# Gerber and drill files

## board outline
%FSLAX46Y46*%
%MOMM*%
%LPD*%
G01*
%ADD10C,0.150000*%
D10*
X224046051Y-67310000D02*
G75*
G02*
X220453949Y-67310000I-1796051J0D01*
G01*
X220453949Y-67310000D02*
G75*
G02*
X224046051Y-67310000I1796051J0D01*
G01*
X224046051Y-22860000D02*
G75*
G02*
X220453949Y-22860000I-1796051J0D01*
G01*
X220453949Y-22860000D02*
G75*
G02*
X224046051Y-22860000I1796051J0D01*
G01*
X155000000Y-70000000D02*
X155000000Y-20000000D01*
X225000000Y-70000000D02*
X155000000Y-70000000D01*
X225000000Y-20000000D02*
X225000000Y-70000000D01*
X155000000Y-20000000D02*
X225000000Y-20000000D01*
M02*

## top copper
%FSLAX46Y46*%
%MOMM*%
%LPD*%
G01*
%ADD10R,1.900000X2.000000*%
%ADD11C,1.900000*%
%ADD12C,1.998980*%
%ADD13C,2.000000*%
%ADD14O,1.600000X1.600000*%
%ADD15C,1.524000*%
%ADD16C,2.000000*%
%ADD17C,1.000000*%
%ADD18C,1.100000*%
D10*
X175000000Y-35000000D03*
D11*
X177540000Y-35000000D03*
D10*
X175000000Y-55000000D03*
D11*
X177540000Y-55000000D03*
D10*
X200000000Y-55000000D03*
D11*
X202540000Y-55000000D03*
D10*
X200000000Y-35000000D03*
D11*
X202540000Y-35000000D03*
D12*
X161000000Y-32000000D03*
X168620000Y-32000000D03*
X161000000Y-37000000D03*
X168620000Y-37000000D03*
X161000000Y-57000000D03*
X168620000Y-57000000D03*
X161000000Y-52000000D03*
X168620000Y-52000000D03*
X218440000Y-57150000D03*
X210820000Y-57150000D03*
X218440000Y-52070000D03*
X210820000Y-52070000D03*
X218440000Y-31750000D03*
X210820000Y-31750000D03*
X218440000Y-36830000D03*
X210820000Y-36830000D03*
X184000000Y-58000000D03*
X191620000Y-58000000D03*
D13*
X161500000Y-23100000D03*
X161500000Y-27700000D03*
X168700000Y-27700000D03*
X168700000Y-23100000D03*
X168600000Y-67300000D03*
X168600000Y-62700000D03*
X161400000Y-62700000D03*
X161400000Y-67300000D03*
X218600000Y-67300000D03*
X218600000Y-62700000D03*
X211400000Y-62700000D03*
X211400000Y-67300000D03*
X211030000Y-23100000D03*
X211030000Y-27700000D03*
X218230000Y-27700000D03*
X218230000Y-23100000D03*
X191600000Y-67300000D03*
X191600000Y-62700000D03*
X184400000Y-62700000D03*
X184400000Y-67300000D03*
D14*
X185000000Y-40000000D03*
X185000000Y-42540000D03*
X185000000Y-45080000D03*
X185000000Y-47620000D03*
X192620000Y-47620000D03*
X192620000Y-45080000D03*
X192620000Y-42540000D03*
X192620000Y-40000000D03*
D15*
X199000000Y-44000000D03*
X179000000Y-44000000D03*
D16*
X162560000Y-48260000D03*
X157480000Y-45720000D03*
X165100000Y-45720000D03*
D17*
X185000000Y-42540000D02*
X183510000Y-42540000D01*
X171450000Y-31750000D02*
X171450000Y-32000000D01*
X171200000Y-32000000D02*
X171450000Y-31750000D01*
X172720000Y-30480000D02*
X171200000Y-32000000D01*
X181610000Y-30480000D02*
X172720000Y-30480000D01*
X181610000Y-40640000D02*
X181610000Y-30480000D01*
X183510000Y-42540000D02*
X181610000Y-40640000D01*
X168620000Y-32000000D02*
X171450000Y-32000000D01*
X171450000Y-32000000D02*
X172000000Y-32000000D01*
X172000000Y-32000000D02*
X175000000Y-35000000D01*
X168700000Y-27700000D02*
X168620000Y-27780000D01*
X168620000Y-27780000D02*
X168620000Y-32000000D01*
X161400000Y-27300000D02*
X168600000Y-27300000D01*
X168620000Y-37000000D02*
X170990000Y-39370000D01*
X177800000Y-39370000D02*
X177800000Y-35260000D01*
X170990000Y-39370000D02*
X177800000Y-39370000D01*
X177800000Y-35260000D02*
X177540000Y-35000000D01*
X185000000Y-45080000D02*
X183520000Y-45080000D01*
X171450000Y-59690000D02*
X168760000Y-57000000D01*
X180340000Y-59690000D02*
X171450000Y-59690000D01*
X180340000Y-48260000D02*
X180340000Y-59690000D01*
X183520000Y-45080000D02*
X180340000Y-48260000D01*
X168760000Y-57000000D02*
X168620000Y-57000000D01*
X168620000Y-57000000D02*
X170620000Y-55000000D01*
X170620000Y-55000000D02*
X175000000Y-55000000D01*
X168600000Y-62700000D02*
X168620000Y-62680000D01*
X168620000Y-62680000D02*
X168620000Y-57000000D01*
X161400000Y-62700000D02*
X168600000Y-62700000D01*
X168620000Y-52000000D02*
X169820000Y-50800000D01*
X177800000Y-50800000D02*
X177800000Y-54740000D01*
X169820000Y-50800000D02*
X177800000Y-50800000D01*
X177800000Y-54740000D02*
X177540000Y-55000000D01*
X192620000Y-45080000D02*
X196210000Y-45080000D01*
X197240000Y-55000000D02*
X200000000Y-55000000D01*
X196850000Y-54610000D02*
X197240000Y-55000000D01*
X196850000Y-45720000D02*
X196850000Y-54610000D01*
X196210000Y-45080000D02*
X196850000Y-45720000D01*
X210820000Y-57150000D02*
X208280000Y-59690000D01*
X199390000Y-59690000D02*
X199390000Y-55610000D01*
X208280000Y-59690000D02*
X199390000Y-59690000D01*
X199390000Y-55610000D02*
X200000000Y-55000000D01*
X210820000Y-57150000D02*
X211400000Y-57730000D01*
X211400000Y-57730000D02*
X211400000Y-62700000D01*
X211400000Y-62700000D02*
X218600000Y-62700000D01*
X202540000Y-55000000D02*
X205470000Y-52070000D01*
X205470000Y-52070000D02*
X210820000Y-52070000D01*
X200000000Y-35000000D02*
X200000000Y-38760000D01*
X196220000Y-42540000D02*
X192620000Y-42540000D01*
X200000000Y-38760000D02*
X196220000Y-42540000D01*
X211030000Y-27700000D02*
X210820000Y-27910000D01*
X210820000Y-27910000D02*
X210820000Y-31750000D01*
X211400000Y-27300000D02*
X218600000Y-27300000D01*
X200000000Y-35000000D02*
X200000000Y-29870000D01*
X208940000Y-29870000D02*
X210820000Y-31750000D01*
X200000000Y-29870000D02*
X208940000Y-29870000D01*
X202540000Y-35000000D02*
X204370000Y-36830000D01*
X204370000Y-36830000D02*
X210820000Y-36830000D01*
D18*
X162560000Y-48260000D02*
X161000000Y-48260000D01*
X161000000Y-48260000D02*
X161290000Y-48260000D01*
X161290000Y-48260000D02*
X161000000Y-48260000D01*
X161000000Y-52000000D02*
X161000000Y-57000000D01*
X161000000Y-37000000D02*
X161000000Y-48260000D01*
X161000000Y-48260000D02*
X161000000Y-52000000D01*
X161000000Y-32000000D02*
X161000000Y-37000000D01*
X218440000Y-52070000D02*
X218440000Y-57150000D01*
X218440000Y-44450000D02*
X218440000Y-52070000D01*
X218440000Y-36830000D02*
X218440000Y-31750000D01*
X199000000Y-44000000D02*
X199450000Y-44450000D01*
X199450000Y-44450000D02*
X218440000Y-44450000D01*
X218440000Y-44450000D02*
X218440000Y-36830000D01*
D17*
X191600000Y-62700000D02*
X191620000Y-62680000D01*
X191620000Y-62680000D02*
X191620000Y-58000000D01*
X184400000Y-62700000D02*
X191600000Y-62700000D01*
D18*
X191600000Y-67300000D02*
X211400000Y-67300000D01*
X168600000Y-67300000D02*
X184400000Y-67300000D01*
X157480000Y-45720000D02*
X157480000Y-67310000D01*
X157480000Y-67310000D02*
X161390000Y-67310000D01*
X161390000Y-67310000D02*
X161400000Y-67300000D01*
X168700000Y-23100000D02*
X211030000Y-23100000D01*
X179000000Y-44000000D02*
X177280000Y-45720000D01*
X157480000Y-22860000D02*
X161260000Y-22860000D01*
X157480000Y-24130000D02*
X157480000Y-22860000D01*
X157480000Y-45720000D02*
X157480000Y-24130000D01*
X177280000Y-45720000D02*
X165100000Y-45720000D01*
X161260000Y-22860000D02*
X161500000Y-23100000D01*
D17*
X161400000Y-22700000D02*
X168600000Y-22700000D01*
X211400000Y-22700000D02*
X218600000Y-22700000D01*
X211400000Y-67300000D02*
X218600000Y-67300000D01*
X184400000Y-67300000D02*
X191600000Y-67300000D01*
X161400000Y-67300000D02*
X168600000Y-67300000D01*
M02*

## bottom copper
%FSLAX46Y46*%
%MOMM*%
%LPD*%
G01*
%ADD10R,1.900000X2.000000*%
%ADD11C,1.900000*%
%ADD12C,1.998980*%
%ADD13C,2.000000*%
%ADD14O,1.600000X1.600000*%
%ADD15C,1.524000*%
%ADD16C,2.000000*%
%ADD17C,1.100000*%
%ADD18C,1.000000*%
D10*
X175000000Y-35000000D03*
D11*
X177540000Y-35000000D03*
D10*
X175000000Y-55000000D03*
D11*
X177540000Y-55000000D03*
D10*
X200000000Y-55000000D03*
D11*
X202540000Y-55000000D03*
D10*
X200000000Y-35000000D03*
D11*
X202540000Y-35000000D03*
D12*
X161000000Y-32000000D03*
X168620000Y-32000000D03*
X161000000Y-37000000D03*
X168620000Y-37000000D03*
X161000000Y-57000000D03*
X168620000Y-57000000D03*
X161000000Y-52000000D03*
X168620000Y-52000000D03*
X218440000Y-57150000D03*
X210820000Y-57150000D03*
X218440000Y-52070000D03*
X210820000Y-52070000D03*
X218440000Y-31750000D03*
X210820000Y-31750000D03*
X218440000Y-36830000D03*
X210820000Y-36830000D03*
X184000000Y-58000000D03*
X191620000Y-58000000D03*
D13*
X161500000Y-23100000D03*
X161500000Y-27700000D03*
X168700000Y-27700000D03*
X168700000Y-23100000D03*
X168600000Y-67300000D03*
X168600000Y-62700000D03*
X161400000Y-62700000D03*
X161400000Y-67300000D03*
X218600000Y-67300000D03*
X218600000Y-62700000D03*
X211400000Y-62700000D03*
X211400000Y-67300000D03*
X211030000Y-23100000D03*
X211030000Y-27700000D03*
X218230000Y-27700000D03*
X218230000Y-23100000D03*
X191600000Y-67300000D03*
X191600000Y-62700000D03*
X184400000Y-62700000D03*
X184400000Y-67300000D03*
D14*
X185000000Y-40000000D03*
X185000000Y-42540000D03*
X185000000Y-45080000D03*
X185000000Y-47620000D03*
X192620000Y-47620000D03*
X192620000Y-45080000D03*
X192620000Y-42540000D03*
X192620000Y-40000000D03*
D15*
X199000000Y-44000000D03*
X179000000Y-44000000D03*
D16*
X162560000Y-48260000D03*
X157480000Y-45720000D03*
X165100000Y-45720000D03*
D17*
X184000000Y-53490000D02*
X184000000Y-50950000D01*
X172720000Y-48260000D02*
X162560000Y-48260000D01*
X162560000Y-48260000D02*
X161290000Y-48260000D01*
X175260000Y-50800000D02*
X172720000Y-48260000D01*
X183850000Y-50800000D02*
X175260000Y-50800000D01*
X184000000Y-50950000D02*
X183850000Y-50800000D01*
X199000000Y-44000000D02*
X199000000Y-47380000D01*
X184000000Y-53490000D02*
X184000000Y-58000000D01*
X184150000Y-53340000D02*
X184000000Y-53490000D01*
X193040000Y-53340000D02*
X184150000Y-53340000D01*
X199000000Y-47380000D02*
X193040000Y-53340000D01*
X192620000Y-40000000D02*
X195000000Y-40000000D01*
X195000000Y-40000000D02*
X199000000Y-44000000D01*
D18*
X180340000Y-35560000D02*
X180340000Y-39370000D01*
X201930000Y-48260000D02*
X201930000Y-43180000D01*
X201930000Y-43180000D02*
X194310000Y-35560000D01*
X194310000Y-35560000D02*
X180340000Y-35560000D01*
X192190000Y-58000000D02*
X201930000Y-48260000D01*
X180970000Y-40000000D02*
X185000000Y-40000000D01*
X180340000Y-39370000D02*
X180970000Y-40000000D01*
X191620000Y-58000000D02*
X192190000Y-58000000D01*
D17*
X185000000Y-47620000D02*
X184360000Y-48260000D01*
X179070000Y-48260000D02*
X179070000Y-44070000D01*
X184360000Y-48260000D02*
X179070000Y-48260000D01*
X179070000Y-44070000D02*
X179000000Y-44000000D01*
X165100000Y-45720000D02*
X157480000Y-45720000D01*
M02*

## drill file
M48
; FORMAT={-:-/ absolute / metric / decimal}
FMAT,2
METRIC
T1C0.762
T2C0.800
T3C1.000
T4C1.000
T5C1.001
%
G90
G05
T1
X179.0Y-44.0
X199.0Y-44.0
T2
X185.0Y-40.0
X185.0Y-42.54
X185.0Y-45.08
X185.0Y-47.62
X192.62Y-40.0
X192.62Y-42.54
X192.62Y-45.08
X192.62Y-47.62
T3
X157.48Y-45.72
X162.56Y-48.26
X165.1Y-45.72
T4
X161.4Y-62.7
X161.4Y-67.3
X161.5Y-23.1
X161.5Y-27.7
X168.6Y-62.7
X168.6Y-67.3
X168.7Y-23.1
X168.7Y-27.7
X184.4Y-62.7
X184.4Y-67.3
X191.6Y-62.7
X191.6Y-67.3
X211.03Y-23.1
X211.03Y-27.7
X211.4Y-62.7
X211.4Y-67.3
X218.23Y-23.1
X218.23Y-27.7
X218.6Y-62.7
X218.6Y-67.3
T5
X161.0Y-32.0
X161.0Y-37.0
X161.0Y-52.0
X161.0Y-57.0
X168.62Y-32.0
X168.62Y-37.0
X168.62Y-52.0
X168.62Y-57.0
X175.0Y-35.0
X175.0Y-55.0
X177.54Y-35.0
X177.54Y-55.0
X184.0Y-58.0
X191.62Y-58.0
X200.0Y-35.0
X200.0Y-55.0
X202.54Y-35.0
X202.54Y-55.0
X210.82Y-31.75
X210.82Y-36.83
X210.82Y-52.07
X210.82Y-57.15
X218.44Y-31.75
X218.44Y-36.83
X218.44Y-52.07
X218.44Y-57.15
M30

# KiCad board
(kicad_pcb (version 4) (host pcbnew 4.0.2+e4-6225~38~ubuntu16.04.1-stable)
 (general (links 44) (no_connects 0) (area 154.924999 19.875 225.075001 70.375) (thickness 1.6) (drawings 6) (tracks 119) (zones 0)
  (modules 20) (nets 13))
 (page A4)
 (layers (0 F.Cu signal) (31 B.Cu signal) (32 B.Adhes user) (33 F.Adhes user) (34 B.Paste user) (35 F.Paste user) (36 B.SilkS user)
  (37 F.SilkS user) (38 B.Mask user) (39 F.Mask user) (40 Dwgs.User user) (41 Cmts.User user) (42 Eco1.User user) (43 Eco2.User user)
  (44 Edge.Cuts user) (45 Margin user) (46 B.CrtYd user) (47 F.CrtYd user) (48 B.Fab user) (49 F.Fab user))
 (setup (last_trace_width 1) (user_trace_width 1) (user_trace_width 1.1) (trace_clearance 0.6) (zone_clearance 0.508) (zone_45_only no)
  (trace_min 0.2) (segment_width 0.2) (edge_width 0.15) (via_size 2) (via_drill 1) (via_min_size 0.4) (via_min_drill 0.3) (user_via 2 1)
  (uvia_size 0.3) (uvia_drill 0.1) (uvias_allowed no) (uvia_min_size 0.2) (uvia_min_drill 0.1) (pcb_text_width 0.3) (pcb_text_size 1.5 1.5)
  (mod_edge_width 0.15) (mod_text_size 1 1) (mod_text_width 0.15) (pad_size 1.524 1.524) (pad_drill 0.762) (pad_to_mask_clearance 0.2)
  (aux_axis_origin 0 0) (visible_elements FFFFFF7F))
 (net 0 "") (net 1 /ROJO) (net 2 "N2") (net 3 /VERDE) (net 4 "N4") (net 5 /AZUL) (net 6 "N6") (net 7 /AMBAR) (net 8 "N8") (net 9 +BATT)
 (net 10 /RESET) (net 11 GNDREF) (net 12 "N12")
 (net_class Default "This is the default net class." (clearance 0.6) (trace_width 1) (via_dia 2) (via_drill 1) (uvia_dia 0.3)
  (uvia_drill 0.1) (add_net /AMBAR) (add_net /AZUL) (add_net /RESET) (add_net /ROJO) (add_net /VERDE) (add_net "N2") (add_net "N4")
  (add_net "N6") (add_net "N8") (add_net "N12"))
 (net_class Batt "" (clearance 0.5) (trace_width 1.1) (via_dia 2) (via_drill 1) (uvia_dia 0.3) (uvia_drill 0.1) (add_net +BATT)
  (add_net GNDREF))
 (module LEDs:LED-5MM (layer F.Cu) (at 175 35)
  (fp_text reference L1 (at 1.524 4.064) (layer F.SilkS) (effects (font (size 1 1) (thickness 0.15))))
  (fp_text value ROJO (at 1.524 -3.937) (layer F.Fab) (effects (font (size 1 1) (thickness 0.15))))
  (pad 1 thru_hole rect (at 0 0 90) (size 2 1.9) (drill 1.00076) (layers *.Cu *.Mask F.SilkS) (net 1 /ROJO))
  (pad 2 thru_hole circle (at 2.54 0) (size 1.9 1.9) (drill 1.00076) (layers *.Cu *.Mask F.SilkS) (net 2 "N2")))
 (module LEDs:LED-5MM (layer F.Cu) (at 175 55)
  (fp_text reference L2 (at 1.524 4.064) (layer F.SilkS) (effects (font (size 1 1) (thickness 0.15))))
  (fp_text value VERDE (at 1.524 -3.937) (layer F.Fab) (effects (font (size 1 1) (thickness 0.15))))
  (pad 1 thru_hole rect (at 0 0 90) (size 2 1.9) (drill 1.00076) (layers *.Cu *.Mask F.SilkS) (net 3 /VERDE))
  (pad 2 thru_hole circle (at 2.54 0) (size 1.9 1.9) (drill 1.00076) (layers *.Cu *.Mask F.SilkS) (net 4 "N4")))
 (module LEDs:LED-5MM (layer F.Cu) (at 200 55)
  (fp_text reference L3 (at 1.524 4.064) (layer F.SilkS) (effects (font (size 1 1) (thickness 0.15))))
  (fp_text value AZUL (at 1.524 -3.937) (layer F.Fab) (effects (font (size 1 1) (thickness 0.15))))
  (pad 1 thru_hole rect (at 0 0 90) (size 2 1.9) (drill 1.00076) (layers *.Cu *.Mask F.SilkS) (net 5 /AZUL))
  (pad 2 thru_hole circle (at 2.54 0) (size 1.9 1.9) (drill 1.00076) (layers *.Cu *.Mask F.SilkS) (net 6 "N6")))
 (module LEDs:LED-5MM (layer F.Cu) (at 200 35)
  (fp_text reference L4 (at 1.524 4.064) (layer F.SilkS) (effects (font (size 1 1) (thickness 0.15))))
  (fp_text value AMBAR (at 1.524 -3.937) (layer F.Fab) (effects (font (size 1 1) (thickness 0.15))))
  (pad 1 thru_hole rect (at 0 0 90) (size 2 1.9) (drill 1.00076) (layers *.Cu *.Mask F.SilkS) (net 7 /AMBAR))
  (pad 2 thru_hole circle (at 2.54 0) (size 1.9 1.9) (drill 1.00076) (layers *.Cu *.Mask F.SilkS) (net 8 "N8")))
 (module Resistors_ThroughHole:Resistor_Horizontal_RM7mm (layer F.Cu) (at 161 32)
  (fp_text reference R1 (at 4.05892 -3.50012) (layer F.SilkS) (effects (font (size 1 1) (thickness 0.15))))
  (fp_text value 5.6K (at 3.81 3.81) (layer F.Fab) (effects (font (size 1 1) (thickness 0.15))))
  (pad 1 thru_hole circle (at 0 0) (size 1.99898 1.99898) (drill 1.00076) (layers *.Cu *.SilkS *.Mask) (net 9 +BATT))
  (pad 2 thru_hole circle (at 7.62 0) (size 1.99898 1.99898) (drill 1.00076) (layers *.Cu *.SilkS *.Mask) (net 1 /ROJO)))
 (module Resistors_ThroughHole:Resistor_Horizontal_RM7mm (layer F.Cu) (at 161 37)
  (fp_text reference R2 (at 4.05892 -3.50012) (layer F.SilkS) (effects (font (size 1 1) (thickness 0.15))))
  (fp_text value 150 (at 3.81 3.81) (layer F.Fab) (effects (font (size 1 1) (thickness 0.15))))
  (pad 1 thru_hole circle (at 0 0) (size 1.99898 1.99898) (drill 1.00076) (layers *.Cu *.SilkS *.Mask) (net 9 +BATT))
  (pad 2 thru_hole circle (at 7.62 0) (size 1.99898 1.99898) (drill 1.00076) (layers *.Cu *.SilkS *.Mask) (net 2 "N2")))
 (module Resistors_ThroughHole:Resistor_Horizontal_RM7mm (layer F.Cu) (at 161 57)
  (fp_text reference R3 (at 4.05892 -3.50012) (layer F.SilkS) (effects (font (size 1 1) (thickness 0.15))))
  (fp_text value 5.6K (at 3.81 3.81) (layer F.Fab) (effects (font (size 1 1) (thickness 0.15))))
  (pad 1 thru_hole circle (at 0 0) (size 1.99898 1.99898) (drill 1.00076) (layers *.Cu *.SilkS *.Mask) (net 9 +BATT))
  (pad 2 thru_hole circle (at 7.62 0) (size 1.99898 1.99898) (drill 1.00076) (layers *.Cu *.SilkS *.Mask) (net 3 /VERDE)))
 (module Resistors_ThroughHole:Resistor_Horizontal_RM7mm (layer F.Cu) (at 161 52)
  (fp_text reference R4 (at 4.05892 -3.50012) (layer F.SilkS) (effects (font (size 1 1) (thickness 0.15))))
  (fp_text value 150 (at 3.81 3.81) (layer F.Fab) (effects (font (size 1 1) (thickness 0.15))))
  (pad 1 thru_hole circle (at 0 0) (size 1.99898 1.99898) (drill 1.00076) (layers *.Cu *.SilkS *.Mask) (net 9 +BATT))
  (pad 2 thru_hole circle (at 7.62 0) (size 1.99898 1.99898) (drill 1.00076) (layers *.Cu *.SilkS *.Mask) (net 4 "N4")))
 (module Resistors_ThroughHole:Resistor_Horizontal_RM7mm (layer F.Cu) (at 218.44 57.15 180)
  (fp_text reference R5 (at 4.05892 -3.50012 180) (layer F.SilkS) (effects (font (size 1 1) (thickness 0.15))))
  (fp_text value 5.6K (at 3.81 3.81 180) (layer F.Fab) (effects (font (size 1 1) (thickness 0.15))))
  (pad 1 thru_hole circle (at 0 0 180) (size 1.99898 1.99898) (drill 1.00076) (layers *.Cu *.SilkS *.Mask) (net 9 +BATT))
  (pad 2 thru_hole circle (at 7.62 0 180) (size 1.99898 1.99898) (drill 1.00076) (layers *.Cu *.SilkS *.Mask) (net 5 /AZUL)))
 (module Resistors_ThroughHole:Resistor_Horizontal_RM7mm (layer F.Cu) (at 218.44 52.07 180)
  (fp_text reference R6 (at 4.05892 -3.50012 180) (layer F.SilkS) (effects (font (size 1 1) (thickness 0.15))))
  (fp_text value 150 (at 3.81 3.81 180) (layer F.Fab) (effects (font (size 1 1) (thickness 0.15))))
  (pad 1 thru_hole circle (at 0 0 180) (size 1.99898 1.99898) (drill 1.00076) (layers *.Cu *.SilkS *.Mask) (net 9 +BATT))
  (pad 2 thru_hole circle (at 7.62 0 180) (size 1.99898 1.99898) (drill 1.00076) (layers *.Cu *.SilkS *.Mask) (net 6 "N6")))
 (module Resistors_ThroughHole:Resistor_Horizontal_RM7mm (layer F.Cu) (at 218.44 31.75 180)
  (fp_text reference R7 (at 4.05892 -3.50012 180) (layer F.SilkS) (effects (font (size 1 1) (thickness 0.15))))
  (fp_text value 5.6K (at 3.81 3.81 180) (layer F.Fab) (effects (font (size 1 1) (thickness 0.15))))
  (pad 1 thru_hole circle (at 0 0 180) (size 1.99898 1.99898) (drill 1.00076) (layers *.Cu *.SilkS *.Mask) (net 9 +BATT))
  (pad 2 thru_hole circle (at 7.62 0 180) (size 1.99898 1.99898) (drill 1.00076) (layers *.Cu *.SilkS *.Mask) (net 7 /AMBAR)))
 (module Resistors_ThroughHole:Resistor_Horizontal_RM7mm (layer F.Cu) (at 218.44 36.83 180)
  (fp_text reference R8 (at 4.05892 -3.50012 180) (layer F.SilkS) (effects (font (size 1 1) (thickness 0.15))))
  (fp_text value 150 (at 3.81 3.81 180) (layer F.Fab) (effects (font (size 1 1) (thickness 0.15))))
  (pad 1 thru_hole circle (at 0 0 180) (size 1.99898 1.99898) (drill 1.00076) (layers *.Cu *.SilkS *.Mask) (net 9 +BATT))
  (pad 2 thru_hole circle (at 7.62 0 180) (size 1.99898 1.99898) (drill 1.00076) (layers *.Cu *.SilkS *.Mask) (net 8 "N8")))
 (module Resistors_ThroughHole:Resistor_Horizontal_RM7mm (layer F.Cu) (at 184 58)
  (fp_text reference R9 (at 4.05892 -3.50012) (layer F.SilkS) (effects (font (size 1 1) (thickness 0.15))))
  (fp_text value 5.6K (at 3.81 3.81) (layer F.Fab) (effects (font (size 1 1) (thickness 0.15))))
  (pad 1 thru_hole circle (at 0 0) (size 1.99898 1.99898) (drill 1.00076) (layers *.Cu *.SilkS *.Mask) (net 9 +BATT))
  (pad 2 thru_hole circle (at 7.62 0) (size 1.99898 1.99898) (drill 1.00076) (layers *.Cu *.SilkS *.Mask) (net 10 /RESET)))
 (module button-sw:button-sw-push (layer F.Cu) (at 165.1 25.4 180)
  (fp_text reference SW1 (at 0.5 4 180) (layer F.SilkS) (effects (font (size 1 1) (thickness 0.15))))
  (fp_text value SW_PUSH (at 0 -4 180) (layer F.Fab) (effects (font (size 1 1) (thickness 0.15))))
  (pad 1 thru_hole circle (at 3.6 2.3 180) (size 2 2) (drill 1) (layers *.Cu *.Mask F.SilkS) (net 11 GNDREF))
  (pad 2 thru_hole circle (at 3.6 -2.3 180) (size 2 2) (drill 1) (layers *.Cu *.Mask F.SilkS) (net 1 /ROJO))
  (pad 2 thru_hole circle (at -3.6 -2.3 180) (size 2 2) (drill 1) (layers *.Cu *.Mask F.SilkS) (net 1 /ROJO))
  (pad 1 thru_hole circle (at -3.6 2.3 180) (size 2 2) (drill 1) (layers *.Cu *.Mask F.SilkS) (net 11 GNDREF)))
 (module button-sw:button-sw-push (layer F.Cu) (at 165 65)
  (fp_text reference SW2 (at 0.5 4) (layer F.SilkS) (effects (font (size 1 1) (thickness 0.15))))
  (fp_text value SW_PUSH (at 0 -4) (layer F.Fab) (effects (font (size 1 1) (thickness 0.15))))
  (pad 1 thru_hole circle (at 3.6 2.3) (size 2 2) (drill 1) (layers *.Cu *.Mask F.SilkS) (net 11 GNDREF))
  (pad 2 thru_hole circle (at 3.6 -2.3) (size 2 2) (drill 1) (layers *.Cu *.Mask F.SilkS) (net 3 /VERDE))
  (pad 2 thru_hole circle (at -3.6 -2.3) (size 2 2) (drill 1) (layers *.Cu *.Mask F.SilkS) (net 3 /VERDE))
  (pad 1 thru_hole circle (at -3.6 2.3) (size 2 2) (drill 1) (layers *.Cu *.Mask F.SilkS) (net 11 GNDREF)))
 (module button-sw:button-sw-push (layer F.Cu) (at 215 65)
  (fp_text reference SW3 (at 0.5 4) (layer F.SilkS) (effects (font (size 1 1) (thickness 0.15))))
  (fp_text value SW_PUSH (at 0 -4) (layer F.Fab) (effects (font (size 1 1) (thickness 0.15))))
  (pad 1 thru_hole circle (at 3.6 2.3) (size 2 2) (drill 1) (layers *.Cu *.Mask F.SilkS) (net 11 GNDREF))
  (pad 2 thru_hole circle (at 3.6 -2.3) (size 2 2) (drill 1) (layers *.Cu *.Mask F.SilkS) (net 5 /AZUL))
  (pad 2 thru_hole circle (at -3.6 -2.3) (size 2 2) (drill 1) (layers *.Cu *.Mask F.SilkS) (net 5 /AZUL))
  (pad 1 thru_hole circle (at -3.6 2.3) (size 2 2) (drill 1) (layers *.Cu *.Mask F.SilkS) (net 11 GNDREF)))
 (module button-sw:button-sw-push (layer F.Cu) (at 214.63 25.4 180)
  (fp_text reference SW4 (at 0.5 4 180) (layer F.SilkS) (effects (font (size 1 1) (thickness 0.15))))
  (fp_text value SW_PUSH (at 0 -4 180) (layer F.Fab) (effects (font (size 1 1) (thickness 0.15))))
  (pad 1 thru_hole circle (at 3.6 2.3 180) (size 2 2) (drill 1) (layers *.Cu *.Mask F.SilkS) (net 11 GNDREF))
  (pad 2 thru_hole circle (at 3.6 -2.3 180) (size 2 2) (drill 1) (layers *.Cu *.Mask F.SilkS) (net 7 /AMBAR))
  (pad 2 thru_hole circle (at -3.6 -2.3 180) (size 2 2) (drill 1) (layers *.Cu *.Mask F.SilkS) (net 7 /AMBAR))
  (pad 1 thru_hole circle (at -3.6 2.3 180) (size 2 2) (drill 1) (layers *.Cu *.Mask F.SilkS) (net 11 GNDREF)))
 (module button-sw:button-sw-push (layer F.Cu) (at 188 65)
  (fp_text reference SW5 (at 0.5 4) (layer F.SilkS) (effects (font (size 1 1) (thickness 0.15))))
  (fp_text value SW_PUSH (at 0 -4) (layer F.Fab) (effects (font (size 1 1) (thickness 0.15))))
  (pad 1 thru_hole circle (at 3.6 2.3) (size 2 2) (drill 1) (layers *.Cu *.Mask F.SilkS) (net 11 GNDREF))
  (pad 2 thru_hole circle (at 3.6 -2.3) (size 2 2) (drill 1) (layers *.Cu *.Mask F.SilkS) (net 10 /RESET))
  (pad 2 thru_hole circle (at -3.6 -2.3) (size 2 2) (drill 1) (layers *.Cu *.Mask F.SilkS) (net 10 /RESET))
  (pad 1 thru_hole circle (at -3.6 2.3) (size 2 2) (drill 1) (layers *.Cu *.Mask F.SilkS) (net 11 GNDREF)))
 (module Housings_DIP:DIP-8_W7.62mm (layer F.Cu) (at 185 40)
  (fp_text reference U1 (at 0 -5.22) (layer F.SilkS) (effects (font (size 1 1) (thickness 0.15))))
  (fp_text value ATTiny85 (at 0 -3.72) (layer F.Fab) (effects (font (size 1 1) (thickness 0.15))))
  (pad 1 thru_hole oval (at 0 0) (size 1.6 1.6) (drill 0.8) (layers *.Cu *.Mask F.SilkS) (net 10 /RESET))
  (pad 2 thru_hole oval (at 0 2.54) (size 1.6 1.6) (drill 0.8) (layers *.Cu *.Mask F.SilkS) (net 1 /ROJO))
  (pad 3 thru_hole oval (at 0 5.08) (size 1.6 1.6) (drill 0.8) (layers *.Cu *.Mask F.SilkS) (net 3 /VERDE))
  (pad 4 thru_hole oval (at 0 7.62) (size 1.6 1.6) (drill 0.8) (layers *.Cu *.Mask F.SilkS) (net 11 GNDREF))
  (pad 5 thru_hole oval (at 7.62 7.62) (size 1.6 1.6) (drill 0.8) (layers *.Cu *.Mask F.SilkS) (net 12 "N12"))
  (pad 6 thru_hole oval (at 7.62 5.08) (size 1.6 1.6) (drill 0.8) (layers *.Cu *.Mask F.SilkS) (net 5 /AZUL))
  (pad 7 thru_hole oval (at 7.62 2.54) (size 1.6 1.6) (drill 0.8) (layers *.Cu *.Mask F.SilkS) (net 7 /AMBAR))
  (pad 8 thru_hole oval (at 7.62 0) (size 1.6 1.6) (drill 0.8) (layers *.Cu *.Mask F.SilkS) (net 9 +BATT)))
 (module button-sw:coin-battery (layer B.Cu) (at 189 44)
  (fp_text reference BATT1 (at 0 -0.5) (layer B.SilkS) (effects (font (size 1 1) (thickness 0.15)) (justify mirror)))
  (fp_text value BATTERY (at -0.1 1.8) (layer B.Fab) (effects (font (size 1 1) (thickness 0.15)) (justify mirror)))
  (pad 1 thru_hole circle (at 10 0) (size 1.524 1.524) (drill 0.762) (layers *.Cu *.Mask B.SilkS) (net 9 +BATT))
  (pad 2 thru_hole circle (at -10 0) (size 1.524 1.524) (drill 0.762) (layers *.Cu *.Mask B.SilkS) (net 11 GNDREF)))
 (gr_circle (center 222.25 67.31) (end 223.52 68.58) (layer Edge.Cuts) (width 0.15))
 (gr_circle (center 222.25 22.86) (end 223.52 24.13) (layer Edge.Cuts) (width 0.15))
 (gr_line (start 155 70) (end 155 20) (angle 90) (layer Edge.Cuts) (width 0.15))
 (gr_line (start 225 70) (end 155 70) (angle 90) (layer Edge.Cuts) (width 0.15))
 (gr_line (start 225 20) (end 225 70) (angle 90) (layer Edge.Cuts) (width 0.15))
 (gr_line (start 155 20) (end 225 20) (angle 90) (layer Edge.Cuts) (width 0.15))
 (segment (start 185 42.54) (end 183.51 42.54) (width 1) (layer F.Cu) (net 1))
 (segment (start 171.45 31.75) (end 171.45 32) (width 1) (layer F.Cu) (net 1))
 (segment (start 171.2 32) (end 171.45 31.75) (width 1) (layer F.Cu) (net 1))
 (segment (start 172.72 30.48) (end 171.2 32) (width 1) (layer F.Cu) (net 1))
 (segment (start 181.61 30.48) (end 172.72 30.48) (width 1) (layer F.Cu) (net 1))
 (segment (start 181.61 40.64) (end 181.61 30.48) (width 1) (layer F.Cu) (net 1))
 (segment (start 183.51 42.54) (end 181.61 40.64) (width 1) (layer F.Cu) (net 1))
 (segment (start 168.62 32) (end 171.45 32) (width 1) (layer F.Cu) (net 1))
 (segment (start 171.45 32) (end 172 32) (width 1) (layer F.Cu) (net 1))
 (segment (start 172 32) (end 175 35) (width 1) (layer F.Cu) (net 1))
 (segment (start 168.7 27.7) (end 168.62 27.78) (width 1) (layer F.Cu) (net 1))
 (segment (start 168.62 27.78) (end 168.62 32) (width 1) (layer F.Cu) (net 1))
 (segment (start 161.4 27.3) (end 168.6 27.3) (width 1) (layer F.Cu) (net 1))
 (segment (start 168.62 37) (end 170.99 39.37) (width 1) (layer F.Cu) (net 2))
 (segment (start 177.8 39.37) (end 177.8 35.26) (width 1) (layer F.Cu) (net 2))
 (segment (start 170.99 39.37) (end 177.8 39.37) (width 1) (layer F.Cu) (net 2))
 (segment (start 177.8 35.26) (end 177.54 35) (width 1) (layer F.Cu) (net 2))
 (segment (start 185 45.08) (end 183.52 45.08) (width 1) (layer F.Cu) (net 3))
 (segment (start 171.45 59.69) (end 168.76 57) (width 1) (layer F.Cu) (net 3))
 (segment (start 180.34 59.69) (end 171.45 59.69) (width 1) (layer F.Cu) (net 3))
 (segment (start 180.34 48.26) (end 180.34 59.69) (width 1) (layer F.Cu) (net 3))
 (segment (start 183.52 45.08) (end 180.34 48.26) (width 1) (layer F.Cu) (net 3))
 (segment (start 168.76 57) (end 168.62 57) (width 1) (layer F.Cu) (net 3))
 (segment (start 168.62 57) (end 170.62 55) (width 1) (layer F.Cu) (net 3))
 (segment (start 170.62 55) (end 175 55) (width 1) (layer F.Cu) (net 3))
 (segment (start 168.6 62.7) (end 168.62 62.68) (width 1) (layer F.Cu) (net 3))
 (segment (start 168.62 62.68) (end 168.62 57) (width 1) (layer F.Cu) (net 3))
 (segment (start 161.4 62.7) (end 168.6 62.7) (width 1) (layer F.Cu) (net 3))
 (segment (start 168.62 52) (end 169.82 50.8) (width 1) (layer F.Cu) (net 4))
 (segment (start 177.8 50.8) (end 177.8 54.74) (width 1) (layer F.Cu) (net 4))
 (segment (start 169.82 50.8) (end 177.8 50.8) (width 1) (layer F.Cu) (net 4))
 (segment (start 177.8 54.74) (end 177.54 55) (width 1) (layer F.Cu) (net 4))
 (segment (start 192.62 45.08) (end 196.21 45.08) (width 1) (layer F.Cu) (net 5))
 (segment (start 197.24 55) (end 200 55) (width 1) (layer F.Cu) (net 5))
 (segment (start 196.85 54.61) (end 197.24 55) (width 1) (layer F.Cu) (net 5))
 (segment (start 196.85 45.72) (end 196.85 54.61) (width 1) (layer F.Cu) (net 5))
 (segment (start 196.21 45.08) (end 196.85 45.72) (width 1) (layer F.Cu) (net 5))
 (segment (start 210.82 57.15) (end 208.28 59.69) (width 1) (layer F.Cu) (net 5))
 (segment (start 199.39 59.69) (end 199.39 55.61) (width 1) (layer F.Cu) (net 5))
 (segment (start 208.28 59.69) (end 199.39 59.69) (width 1) (layer F.Cu) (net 5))
 (segment (start 199.39 55.61) (end 200 55) (width 1) (layer F.Cu) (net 5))
 (segment (start 210.82 57.15) (end 211.4 57.73) (width 1) (layer F.Cu) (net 5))
 (segment (start 211.4 57.73) (end 211.4 62.7) (width 1) (layer F.Cu) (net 5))
 (segment (start 211.4 62.7) (end 218.6 62.7) (width 1) (layer F.Cu) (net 5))
 (segment (start 202.54 55) (end 205.47 52.07) (width 1) (layer F.Cu) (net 6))
 (segment (start 205.47 52.07) (end 210.82 52.07) (width 1) (layer F.Cu) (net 6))
 (segment (start 200 35) (end 200 38.76) (width 1) (layer F.Cu) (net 7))
 (segment (start 196.22 42.54) (end 192.62 42.54) (width 1) (layer F.Cu) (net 7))
 (segment (start 200 38.76) (end 196.22 42.54) (width 1) (layer F.Cu) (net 7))
 (segment (start 211.03 27.7) (end 210.82 27.91) (width 1) (layer F.Cu) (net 7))
 (segment (start 210.82 27.91) (end 210.82 31.75) (width 1) (layer F.Cu) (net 7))
 (segment (start 211.4 27.3) (end 218.6 27.3) (width 1) (layer F.Cu) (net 7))
 (segment (start 200 35) (end 200 29.87) (width 1) (layer F.Cu) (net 7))
 (segment (start 208.94 29.87) (end 210.82 31.75) (width 1) (layer F.Cu) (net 7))
 (segment (start 200 29.87) (end 208.94 29.87) (width 1) (layer F.Cu) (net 7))
 (segment (start 202.54 35) (end 204.37 36.83) (width 1) (layer F.Cu) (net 8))
 (segment (start 204.37 36.83) (end 210.82 36.83) (width 1) (layer F.Cu) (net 8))
 (via (at 162.56 48.26) (size 2) (drill 1) (layers F.Cu B.Cu) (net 9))
 (segment (start 162.56 48.26) (end 161 48.26) (width 1.1) (layer F.Cu) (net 9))
 (segment (start 161 48.26) (end 161.29 48.26) (width 1.1) (layer F.Cu) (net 9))
 (segment (start 161.29 48.26) (end 161 48.26) (width 1.1) (layer F.Cu) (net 9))
 (segment (start 184 53.49) (end 184 50.95) (width 1.1) (layer B.Cu) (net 9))
 (segment (start 172.72 48.26) (end 162.56 48.26) (width 1.1) (layer B.Cu) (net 9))
 (segment (start 162.56 48.26) (end 161.29 48.26) (width 1.1) (layer B.Cu) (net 9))
 (segment (start 175.26 50.8) (end 172.72 48.26) (width 1.1) (layer B.Cu) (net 9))
 (segment (start 183.85 50.8) (end 175.26 50.8) (width 1.1) (layer B.Cu) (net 9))
 (segment (start 184 50.95) (end 183.85 50.8) (width 1.1) (layer B.Cu) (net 9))
 (segment (start 199 44) (end 199 47.38) (width 1.1) (layer B.Cu) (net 9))
 (segment (start 184 53.49) (end 184 58) (width 1.1) (layer B.Cu) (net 9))
 (segment (start 184.15 53.34) (end 184 53.49) (width 1.1) (layer B.Cu) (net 9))
 (segment (start 193.04 53.34) (end 184.15 53.34) (width 1.1) (layer B.Cu) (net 9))
 (segment (start 199 47.38) (end 193.04 53.34) (width 1.1) (layer B.Cu) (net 9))
 (segment (start 192.62 40) (end 195 40) (width 1.1) (layer B.Cu) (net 9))
 (segment (start 195 40) (end 199 44) (width 1.1) (layer B.Cu) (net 9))
 (segment (start 161 52) (end 161 57) (width 1.1) (layer F.Cu) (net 9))
 (segment (start 161 37) (end 161 48.26) (width 1.1) (layer F.Cu) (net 9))
 (segment (start 161 48.26) (end 161 52) (width 1.1) (layer F.Cu) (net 9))
 (segment (start 161 32) (end 161 37) (width 1.1) (layer F.Cu) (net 9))
 (segment (start 218.44 52.07) (end 218.44 57.15) (width 1.1) (layer F.Cu) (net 9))
 (segment (start 218.44 44.45) (end 218.44 52.07) (width 1.1) (layer F.Cu) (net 9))
 (segment (start 218.44 36.83) (end 218.44 31.75) (width 1.1) (layer F.Cu) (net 9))
 (segment (start 199 44) (end 199.45 44.45) (width 1.1) (layer F.Cu) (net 9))
 (segment (start 199.45 44.45) (end 218.44 44.45) (width 1.1) (layer F.Cu) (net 9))
 (segment (start 218.44 44.45) (end 218.44 36.83) (width 1.1) (layer F.Cu) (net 9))
 (segment (start 180.34 35.56) (end 180.34 39.37) (width 1) (layer B.Cu) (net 10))
 (segment (start 201.93 48.26) (end 201.93 43.18) (width 1) (layer B.Cu) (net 10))
 (segment (start 201.93 43.18) (end 194.31 35.56) (width 1) (layer B.Cu) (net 10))
 (segment (start 194.31 35.56) (end 180.34 35.56) (width 1) (layer B.Cu) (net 10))
 (segment (start 192.19 58) (end 201.93 48.26) (width 1) (layer B.Cu) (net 10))
 (segment (start 180.97 40) (end 185 40) (width 1) (layer B.Cu) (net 10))
 (segment (start 180.34 39.37) (end 180.97 40) (width 1) (layer B.Cu) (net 10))
 (segment (start 191.62 58) (end 192.19 58) (width 1) (layer B.Cu) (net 10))
 (segment (start 191.6 62.7) (end 191.62 62.68) (width 1) (layer F.Cu) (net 10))
 (segment (start 191.62 62.68) (end 191.62 58) (width 1) (layer F.Cu) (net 10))
 (segment (start 184.4 62.7) (end 191.6 62.7) (width 1) (layer F.Cu) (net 10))
 (segment (start 185 47.62) (end 184.36 48.26) (width 1.1) (layer B.Cu) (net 11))
 (segment (start 179.07 48.26) (end 179.07 44.07) (width 1.1) (layer B.Cu) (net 11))
 (segment (start 184.36 48.26) (end 179.07 48.26) (width 1.1) (layer B.Cu) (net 11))
 (segment (start 179.07 44.07) (end 179 44) (width 1.1) (layer B.Cu) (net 11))
 (segment (start 191.6 67.3) (end 211.4 67.3) (width 1.1) (layer F.Cu) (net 11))
 (segment (start 168.6 67.3) (end 184.4 67.3) (width 1.1) (layer F.Cu) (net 11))
 (segment (start 157.48 45.72) (end 157.48 67.31) (width 1.1) (layer F.Cu) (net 11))
 (segment (start 157.48 67.31) (end 161.39 67.31) (width 1.1) (layer F.Cu) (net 11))
 (segment (start 161.39 67.31) (end 161.4 67.3) (width 1.1) (layer F.Cu) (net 11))
 (segment (start 168.7 23.1) (end 211.03 23.1) (width 1.1) (layer F.Cu) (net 11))
 (segment (start 179 44) (end 177.28 45.72) (width 1.1) (layer F.Cu) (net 11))
 (segment (start 157.48 22.86) (end 161.26 22.86) (width 1.1) (layer F.Cu) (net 11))
 (segment (start 157.48 24.13) (end 157.48 22.86) (width 1.1) (layer F.Cu) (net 11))
 (segment (start 157.48 45.72) (end 157.48 24.13) (width 1.1) (layer F.Cu) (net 11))
 (via (at 157.48 45.72) (size 2) (drill 1) (layers F.Cu B.Cu) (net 11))
 (segment (start 165.1 45.72) (end 157.48 45.72) (width 1.1) (layer B.Cu) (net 11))
 (via (at 165.1 45.72) (size 2) (drill 1) (layers F.Cu B.Cu) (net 11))
 (segment (start 177.28 45.72) (end 165.1 45.72) (width 1.1) (layer F.Cu) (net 11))
 (segment (start 161.26 22.86) (end 161.5 23.1) (width 1.1) (layer F.Cu) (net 11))
 (segment (start 161.4 22.7) (end 168.6 22.7) (width 1) (layer F.Cu) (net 11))
 (segment (start 211.4 22.7) (end 218.6 22.7) (width 1) (layer F.Cu) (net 11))
 (segment (start 211.4 67.3) (end 218.6 67.3) (width 1) (layer F.Cu) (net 11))
 (segment (start 184.4 67.3) (end 191.6 67.3) (width 1) (layer F.Cu) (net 11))
 (segment (start 161.4 67.3) (end 168.6 67.3) (width 1) (layer F.Cu) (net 11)))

